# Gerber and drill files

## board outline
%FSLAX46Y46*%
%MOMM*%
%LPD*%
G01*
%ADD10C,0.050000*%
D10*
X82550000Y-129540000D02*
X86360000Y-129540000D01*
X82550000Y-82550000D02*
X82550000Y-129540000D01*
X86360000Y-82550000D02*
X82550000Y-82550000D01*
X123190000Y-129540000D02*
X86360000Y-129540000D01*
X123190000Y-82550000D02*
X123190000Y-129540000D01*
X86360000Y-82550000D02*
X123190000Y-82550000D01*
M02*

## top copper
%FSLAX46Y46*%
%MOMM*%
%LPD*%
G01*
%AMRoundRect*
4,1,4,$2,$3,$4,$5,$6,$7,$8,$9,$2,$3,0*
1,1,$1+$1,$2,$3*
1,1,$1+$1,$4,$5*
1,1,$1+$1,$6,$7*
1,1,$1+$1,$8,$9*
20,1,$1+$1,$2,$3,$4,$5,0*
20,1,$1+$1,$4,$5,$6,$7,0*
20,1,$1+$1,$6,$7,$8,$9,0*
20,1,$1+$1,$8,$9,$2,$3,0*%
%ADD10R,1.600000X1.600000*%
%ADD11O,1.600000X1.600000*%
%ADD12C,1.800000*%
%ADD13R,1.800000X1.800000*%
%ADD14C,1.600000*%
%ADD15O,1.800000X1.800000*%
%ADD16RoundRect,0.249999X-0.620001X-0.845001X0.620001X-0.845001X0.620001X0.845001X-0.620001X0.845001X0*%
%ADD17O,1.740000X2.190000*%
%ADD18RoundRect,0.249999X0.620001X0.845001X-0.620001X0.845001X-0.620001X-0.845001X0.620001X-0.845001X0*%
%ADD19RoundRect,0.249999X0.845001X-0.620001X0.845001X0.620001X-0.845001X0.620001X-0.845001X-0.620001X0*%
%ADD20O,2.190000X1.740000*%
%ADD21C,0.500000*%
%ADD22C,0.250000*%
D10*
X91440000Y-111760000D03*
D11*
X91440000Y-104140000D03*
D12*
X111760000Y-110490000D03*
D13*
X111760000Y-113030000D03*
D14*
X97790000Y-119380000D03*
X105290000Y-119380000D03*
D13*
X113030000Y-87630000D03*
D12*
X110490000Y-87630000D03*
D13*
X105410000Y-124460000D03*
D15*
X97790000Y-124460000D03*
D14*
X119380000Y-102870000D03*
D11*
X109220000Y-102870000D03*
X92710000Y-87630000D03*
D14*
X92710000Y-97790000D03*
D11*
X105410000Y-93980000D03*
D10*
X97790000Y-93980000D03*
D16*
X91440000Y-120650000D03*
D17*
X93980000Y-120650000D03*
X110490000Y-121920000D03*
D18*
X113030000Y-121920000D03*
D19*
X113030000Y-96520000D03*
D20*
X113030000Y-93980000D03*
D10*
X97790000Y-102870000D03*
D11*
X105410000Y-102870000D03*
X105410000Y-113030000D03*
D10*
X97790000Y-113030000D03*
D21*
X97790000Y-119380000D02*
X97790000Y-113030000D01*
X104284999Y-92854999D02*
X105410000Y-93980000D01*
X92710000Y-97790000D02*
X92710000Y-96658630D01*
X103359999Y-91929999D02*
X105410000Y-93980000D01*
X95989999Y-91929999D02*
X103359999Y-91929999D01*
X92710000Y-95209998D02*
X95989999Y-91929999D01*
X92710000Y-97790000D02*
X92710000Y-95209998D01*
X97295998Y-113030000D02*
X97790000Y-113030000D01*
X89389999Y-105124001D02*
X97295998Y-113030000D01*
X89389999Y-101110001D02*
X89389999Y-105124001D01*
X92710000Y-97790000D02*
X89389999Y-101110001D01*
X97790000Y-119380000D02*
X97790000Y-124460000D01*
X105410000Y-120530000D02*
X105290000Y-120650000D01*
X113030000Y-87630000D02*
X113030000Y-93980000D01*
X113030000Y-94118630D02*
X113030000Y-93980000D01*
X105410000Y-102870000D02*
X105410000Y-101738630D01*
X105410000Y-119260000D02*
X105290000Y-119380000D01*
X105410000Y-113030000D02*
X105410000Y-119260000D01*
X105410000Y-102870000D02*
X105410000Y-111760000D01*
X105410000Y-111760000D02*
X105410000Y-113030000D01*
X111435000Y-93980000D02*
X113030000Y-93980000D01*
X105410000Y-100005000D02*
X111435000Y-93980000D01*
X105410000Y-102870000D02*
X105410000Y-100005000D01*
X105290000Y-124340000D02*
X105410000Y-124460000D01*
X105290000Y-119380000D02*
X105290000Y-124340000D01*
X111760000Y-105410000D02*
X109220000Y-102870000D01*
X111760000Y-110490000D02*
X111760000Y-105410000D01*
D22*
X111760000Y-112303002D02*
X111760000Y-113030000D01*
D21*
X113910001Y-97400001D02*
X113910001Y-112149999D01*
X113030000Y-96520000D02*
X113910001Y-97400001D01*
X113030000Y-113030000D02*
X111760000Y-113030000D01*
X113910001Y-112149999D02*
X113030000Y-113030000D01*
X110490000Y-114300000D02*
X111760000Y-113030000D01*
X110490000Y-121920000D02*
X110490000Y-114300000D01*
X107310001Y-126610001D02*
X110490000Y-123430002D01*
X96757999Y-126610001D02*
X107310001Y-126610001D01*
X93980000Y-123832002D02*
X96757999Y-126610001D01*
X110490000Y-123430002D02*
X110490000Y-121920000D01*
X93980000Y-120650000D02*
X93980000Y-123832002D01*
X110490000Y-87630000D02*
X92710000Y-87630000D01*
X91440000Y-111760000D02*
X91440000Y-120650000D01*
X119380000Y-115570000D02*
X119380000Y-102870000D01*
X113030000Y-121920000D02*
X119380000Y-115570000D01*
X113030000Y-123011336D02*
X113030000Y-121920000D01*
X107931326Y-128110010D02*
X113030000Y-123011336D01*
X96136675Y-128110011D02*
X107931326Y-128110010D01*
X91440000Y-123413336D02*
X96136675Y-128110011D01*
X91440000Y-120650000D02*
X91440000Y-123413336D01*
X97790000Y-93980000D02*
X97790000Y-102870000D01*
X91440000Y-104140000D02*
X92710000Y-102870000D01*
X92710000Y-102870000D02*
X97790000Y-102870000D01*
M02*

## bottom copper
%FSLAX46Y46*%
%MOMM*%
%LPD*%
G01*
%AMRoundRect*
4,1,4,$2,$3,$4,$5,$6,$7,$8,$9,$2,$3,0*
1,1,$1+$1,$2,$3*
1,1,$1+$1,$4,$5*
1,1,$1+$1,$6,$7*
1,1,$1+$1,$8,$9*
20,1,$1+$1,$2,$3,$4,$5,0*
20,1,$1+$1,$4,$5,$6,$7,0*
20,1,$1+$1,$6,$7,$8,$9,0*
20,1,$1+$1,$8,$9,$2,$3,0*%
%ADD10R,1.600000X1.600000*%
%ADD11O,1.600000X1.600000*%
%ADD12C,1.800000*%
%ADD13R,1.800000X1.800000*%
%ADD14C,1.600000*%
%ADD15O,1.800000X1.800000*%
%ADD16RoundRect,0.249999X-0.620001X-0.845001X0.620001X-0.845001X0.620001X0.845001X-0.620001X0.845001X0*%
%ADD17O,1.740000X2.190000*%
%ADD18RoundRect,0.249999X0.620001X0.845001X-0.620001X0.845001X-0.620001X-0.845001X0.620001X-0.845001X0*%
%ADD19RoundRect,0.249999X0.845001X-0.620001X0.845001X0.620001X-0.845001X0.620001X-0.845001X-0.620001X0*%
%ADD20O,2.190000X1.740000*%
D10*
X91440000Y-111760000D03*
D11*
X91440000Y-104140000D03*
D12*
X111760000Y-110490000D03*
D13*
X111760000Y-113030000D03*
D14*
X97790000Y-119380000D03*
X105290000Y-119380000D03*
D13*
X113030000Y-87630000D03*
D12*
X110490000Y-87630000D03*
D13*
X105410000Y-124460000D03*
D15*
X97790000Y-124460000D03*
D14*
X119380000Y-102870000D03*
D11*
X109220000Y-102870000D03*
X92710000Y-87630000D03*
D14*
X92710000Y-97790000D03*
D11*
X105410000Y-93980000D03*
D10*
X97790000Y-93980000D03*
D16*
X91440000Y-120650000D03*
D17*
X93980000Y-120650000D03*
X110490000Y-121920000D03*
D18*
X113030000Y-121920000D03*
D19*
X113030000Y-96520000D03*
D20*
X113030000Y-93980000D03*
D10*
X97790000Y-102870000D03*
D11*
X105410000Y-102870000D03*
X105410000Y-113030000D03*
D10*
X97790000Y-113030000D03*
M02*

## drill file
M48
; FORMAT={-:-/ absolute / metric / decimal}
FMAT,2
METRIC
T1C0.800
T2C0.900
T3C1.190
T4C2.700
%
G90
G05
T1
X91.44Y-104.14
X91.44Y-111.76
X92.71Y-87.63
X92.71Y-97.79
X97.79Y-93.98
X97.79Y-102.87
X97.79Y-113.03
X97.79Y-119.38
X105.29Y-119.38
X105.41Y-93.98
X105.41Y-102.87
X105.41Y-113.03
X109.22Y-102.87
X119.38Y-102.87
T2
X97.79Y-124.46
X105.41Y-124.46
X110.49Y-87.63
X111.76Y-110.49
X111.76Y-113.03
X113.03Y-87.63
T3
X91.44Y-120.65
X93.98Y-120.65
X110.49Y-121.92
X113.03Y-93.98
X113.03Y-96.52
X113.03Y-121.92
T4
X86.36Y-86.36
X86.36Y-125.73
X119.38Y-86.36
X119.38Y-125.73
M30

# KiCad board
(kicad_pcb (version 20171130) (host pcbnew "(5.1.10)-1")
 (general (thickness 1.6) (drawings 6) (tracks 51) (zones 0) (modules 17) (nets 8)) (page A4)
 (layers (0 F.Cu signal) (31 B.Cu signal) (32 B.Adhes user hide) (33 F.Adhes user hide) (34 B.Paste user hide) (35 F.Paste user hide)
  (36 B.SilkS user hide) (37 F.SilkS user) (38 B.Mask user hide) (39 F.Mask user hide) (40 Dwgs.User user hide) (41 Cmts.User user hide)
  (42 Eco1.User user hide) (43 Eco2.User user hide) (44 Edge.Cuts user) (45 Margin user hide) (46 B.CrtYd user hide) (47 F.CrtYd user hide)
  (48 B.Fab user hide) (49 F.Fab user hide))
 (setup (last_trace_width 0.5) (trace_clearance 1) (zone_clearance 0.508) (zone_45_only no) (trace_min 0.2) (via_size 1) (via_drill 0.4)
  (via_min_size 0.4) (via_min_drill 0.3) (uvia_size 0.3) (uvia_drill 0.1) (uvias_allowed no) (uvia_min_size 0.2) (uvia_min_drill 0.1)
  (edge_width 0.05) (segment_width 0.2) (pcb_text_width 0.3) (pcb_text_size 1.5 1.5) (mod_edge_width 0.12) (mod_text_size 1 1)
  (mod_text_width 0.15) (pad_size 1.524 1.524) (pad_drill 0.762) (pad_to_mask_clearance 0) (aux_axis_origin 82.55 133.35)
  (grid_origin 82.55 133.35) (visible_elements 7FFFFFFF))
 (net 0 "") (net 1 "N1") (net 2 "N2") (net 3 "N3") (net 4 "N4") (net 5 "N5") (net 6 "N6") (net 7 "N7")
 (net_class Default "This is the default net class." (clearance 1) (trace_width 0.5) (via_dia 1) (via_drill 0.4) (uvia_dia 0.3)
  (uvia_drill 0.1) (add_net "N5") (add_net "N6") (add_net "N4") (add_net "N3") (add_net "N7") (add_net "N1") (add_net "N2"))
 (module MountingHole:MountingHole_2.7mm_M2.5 (layer F.Cu) (at 86.36 125.73)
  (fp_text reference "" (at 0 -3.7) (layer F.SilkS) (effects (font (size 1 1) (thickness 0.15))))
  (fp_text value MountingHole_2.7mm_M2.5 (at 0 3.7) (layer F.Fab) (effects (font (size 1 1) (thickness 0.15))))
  (pad 1 np_thru_hole circle (at 0 0) (size 2.7 2.7) (drill 2.7) (layers *.Cu *.Mask)))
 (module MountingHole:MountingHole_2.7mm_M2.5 (layer F.Cu) (at 86.36 86.36)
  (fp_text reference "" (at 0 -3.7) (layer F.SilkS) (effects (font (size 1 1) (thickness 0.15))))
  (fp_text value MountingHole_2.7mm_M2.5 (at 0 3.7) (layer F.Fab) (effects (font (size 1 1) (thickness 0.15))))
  (pad 1 np_thru_hole circle (at 0 0) (size 2.7 2.7) (drill 2.7) (layers *.Cu *.Mask)))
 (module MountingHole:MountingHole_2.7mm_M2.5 (layer F.Cu) (at 119.38 125.73)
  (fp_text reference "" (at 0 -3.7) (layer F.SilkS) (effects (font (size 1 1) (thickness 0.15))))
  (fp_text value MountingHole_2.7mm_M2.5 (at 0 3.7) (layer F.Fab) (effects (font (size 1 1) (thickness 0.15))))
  (pad 1 np_thru_hole circle (at 0 0) (size 2.7 2.7) (drill 2.7) (layers *.Cu *.Mask)))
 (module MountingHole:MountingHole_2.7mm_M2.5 (layer F.Cu) (at 119.38 86.36)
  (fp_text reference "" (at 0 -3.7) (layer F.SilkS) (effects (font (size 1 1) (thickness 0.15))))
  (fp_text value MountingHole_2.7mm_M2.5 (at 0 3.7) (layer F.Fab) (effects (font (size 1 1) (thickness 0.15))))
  (pad 1 np_thru_hole circle (at 0 0) (size 2.7 2.7) (drill 2.7) (layers *.Cu *.Mask)))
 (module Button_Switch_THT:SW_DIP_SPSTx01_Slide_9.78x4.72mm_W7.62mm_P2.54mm (layer F.Cu) (at 91.44 111.76 90)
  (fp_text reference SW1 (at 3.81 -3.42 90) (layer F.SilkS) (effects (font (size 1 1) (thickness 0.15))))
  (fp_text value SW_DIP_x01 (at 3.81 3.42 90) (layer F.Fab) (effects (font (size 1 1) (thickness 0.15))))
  (pad 1 thru_hole rect (at 0 0 90) (size 1.6 1.6) (drill 0.8) (layers *.Cu *.Mask) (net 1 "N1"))
  (pad 2 thru_hole oval (at 7.62 0 90) (size 1.6 1.6) (drill 0.8) (layers *.Cu *.Mask) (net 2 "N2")))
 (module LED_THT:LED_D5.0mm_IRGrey (layer F.Cu) (at 111.76 113.03 90)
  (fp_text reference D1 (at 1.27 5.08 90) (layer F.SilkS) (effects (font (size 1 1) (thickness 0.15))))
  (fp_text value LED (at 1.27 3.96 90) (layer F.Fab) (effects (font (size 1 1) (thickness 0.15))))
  (pad 2 thru_hole circle (at 2.54 0 90) (size 1.8 1.8) (drill 0.9) (layers *.Cu *.Mask) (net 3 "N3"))
  (pad 1 thru_hole rect (at 0 0 90) (size 1.8 1.8) (drill 0.9) (layers *.Cu *.Mask) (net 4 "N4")))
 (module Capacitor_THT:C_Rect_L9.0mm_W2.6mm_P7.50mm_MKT (layer F.Cu) (at 97.79 119.38)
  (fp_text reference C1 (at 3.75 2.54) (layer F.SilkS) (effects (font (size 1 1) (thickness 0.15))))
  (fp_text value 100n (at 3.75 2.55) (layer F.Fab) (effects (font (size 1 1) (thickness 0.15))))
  (pad 1 thru_hole circle (at 0 0) (size 1.6 1.6) (drill 0.8) (layers *.Cu *.Mask) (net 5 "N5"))
  (pad 2 thru_hole circle (at 7.5 0) (size 1.6 1.6) (drill 0.8) (layers *.Cu *.Mask) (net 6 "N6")))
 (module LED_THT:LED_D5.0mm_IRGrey (layer F.Cu) (at 113.03 87.63 180)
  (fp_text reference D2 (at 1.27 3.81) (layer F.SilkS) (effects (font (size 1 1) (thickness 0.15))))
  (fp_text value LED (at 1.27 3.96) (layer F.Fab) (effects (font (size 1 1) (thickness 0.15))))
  (pad 1 thru_hole rect (at 0 0 180) (size 1.8 1.8) (drill 0.9) (layers *.Cu *.Mask) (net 6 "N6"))
  (pad 2 thru_hole circle (at 2.54 0 180) (size 1.8 1.8) (drill 0.9) (layers *.Cu *.Mask) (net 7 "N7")))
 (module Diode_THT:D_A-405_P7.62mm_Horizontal (layer F.Cu) (at 105.41 124.46 180)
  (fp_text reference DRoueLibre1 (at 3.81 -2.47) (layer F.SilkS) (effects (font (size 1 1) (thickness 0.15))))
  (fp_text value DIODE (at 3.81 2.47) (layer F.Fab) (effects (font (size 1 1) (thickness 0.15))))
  (pad 1 thru_hole rect (at 0 0 180) (size 1.8 1.8) (drill 0.9) (layers *.Cu *.Mask) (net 6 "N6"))
  (pad 2 thru_hole oval (at 7.62 0 180) (size 1.8 1.8) (drill 0.9) (layers *.Cu *.Mask) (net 5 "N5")))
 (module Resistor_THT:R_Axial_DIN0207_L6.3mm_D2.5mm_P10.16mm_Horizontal (layer F.Cu) (at 119.38 102.87 180)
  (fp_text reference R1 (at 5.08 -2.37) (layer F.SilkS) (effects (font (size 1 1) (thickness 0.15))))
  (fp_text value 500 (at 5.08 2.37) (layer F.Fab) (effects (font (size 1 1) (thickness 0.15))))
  (pad 1 thru_hole circle (at 0 0 180) (size 1.6 1.6) (drill 0.8) (layers *.Cu *.Mask) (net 1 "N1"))
  (pad 2 thru_hole oval (at 10.16 0 180) (size 1.6 1.6) (drill 0.8) (layers *.Cu *.Mask) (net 3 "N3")))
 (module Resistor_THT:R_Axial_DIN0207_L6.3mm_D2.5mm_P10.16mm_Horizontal (layer F.Cu) (at 92.71 97.79 90)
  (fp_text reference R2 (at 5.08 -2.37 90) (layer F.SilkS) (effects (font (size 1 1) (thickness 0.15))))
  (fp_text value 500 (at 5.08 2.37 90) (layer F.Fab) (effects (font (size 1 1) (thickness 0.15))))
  (pad 2 thru_hole oval (at 10.16 0 90) (size 1.6 1.6) (drill 0.8) (layers *.Cu *.Mask) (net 7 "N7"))
  (pad 1 thru_hole circle (at 0 0 90) (size 1.6 1.6) (drill 0.8) (layers *.Cu *.Mask) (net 5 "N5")))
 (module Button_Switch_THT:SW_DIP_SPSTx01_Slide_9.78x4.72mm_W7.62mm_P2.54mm (layer F.Cu) (at 97.79 93.98)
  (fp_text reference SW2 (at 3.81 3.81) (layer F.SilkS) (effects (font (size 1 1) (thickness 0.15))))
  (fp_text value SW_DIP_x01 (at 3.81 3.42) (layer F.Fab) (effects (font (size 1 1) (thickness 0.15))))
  (pad 2 thru_hole oval (at 7.62 0) (size 1.6 1.6) (drill 0.8) (layers *.Cu *.Mask) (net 5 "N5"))
  (pad 1 thru_hole rect (at 0 0) (size 1.6 1.6) (drill 0.8) (layers *.Cu *.Mask) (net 2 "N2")))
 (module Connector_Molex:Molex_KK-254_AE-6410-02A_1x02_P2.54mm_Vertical (layer F.Cu) (at 91.44 120.65)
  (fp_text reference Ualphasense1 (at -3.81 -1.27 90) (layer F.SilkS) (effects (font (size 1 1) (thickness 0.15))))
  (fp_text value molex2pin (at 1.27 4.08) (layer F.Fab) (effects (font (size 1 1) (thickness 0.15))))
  (pad 1 thru_hole roundrect (at 0 0) (size 1.74 2.19) (drill 1.19) (layers *.Cu *.Mask) (roundrect_rratio 0.1436775862068966) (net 1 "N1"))
  (pad 2 thru_hole oval (at 2.54 0) (size 1.74 2.19) (drill 1.19) (layers *.Cu *.Mask) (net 4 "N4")))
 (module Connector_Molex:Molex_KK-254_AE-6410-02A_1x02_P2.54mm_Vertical (layer F.Cu) (at 113.03 121.92 180)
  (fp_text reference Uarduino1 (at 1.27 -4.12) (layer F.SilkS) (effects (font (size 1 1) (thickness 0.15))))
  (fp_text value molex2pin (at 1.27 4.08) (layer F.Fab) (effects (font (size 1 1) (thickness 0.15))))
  (pad 2 thru_hole oval (at 2.54 0 180) (size 1.74 2.19) (drill 1.19) (layers *.Cu *.Mask) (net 4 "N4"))
  (pad 1 thru_hole roundrect (at 0 0 180) (size 1.74 2.19) (drill 1.19) (layers *.Cu *.Mask) (roundrect_rratio 0.1436775862068966)
   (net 1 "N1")))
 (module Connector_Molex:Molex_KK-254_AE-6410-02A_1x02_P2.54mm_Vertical (layer F.Cu) (at 113.03 96.52 90)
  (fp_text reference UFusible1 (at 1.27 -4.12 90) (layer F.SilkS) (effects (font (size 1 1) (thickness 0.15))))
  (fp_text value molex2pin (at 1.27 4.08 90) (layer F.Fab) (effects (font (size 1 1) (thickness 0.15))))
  (pad 1 thru_hole roundrect (at 0 0 90) (size 1.74 2.19) (drill 1.19) (layers *.Cu *.Mask) (roundrect_rratio 0.1436775862068966)
   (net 4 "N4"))
  (pad 2 thru_hole oval (at 2.54 0 90) (size 1.74 2.19) (drill 1.19) (layers *.Cu *.Mask) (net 6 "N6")))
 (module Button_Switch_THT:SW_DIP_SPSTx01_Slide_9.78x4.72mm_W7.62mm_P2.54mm (layer F.Cu) (at 97.79 102.87)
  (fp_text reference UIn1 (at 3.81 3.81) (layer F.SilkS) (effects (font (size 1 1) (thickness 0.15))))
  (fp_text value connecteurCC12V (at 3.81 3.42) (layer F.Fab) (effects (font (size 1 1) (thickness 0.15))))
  (pad 1 thru_hole rect (at 0 0) (size 1.6 1.6) (drill 0.8) (layers *.Cu *.Mask) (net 2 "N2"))
  (pad 2 thru_hole oval (at 7.62 0) (size 1.6 1.6) (drill 0.8) (layers *.Cu *.Mask) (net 6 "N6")))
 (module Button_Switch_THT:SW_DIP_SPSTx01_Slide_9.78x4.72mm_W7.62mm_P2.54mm (layer F.Cu) (at 97.79 113.03)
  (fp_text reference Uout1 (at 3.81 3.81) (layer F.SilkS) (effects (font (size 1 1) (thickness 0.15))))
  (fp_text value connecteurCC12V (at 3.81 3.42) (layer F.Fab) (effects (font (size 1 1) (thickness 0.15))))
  (pad 2 thru_hole oval (at 7.62 0) (size 1.6 1.6) (drill 0.8) (layers *.Cu *.Mask) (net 6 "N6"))
  (pad 1 thru_hole rect (at 0 0) (size 1.6 1.6) (drill 0.8) (layers *.Cu *.Mask) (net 5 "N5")))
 (gr_line (start 82.55 129.54) (end 86.36 129.54) (layer Edge.Cuts) (width 0.05))
 (gr_line (start 82.55 82.55) (end 82.55 129.54) (layer Edge.Cuts) (width 0.05))
 (gr_line (start 86.36 82.55) (end 82.55 82.55) (layer Edge.Cuts) (width 0.05))
 (gr_line (start 123.19 129.54) (end 86.36 129.54) (layer Edge.Cuts) (width 0.05))
 (gr_line (start 123.19 82.55) (end 123.19 129.54) (layer Edge.Cuts) (width 0.05))
 (gr_line (start 86.36 82.55) (end 123.19 82.55) (layer Edge.Cuts) (width 0.05))
 (segment (start 97.79 119.38) (end 97.79 113.03) (width 0.5) (layer F.Cu) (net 5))
 (segment (start 104.284999 92.854999) (end 105.41 93.98) (width 0.5) (layer F.Cu) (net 5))
 (segment (start 92.71 97.79) (end 92.71 96.65863) (width 0.5) (layer F.Cu) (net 5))
 (segment (start 103.359999 91.929999) (end 105.41 93.98) (width 0.5) (layer F.Cu) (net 5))
 (segment (start 95.989999 91.929999) (end 103.359999 91.929999) (width 0.5) (layer F.Cu) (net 5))
 (segment (start 92.71 95.209998) (end 95.989999 91.929999) (width 0.5) (layer F.Cu) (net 5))
 (segment (start 92.71 97.79) (end 92.71 95.209998) (width 0.5) (layer F.Cu) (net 5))
 (segment (start 97.295998 113.03) (end 97.79 113.03) (width 0.5) (layer F.Cu) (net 5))
 (segment (start 89.389999 105.124001) (end 97.295998 113.03) (width 0.5) (layer F.Cu) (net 5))
 (segment (start 89.389999 101.110001) (end 89.389999 105.124001) (width 0.5) (layer F.Cu) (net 5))
 (segment (start 92.71 97.79) (end 89.389999 101.110001) (width 0.5) (layer F.Cu) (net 5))
 (segment (start 97.79 119.38) (end 97.79 124.46) (width 0.5) (layer F.Cu) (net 5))
 (segment (start 105.41 120.53) (end 105.29 120.65) (width 0.5) (layer F.Cu) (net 6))
 (segment (start 113.03 87.63) (end 113.03 93.98) (width 0.5) (layer F.Cu) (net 6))
 (segment (start 113.03 94.11863) (end 113.03 93.98) (width 0.5) (layer F.Cu) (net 6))
 (segment (start 105.41 102.87) (end 105.41 101.73863) (width 0.5) (layer F.Cu) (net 6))
 (segment (start 105.41 119.26) (end 105.29 119.38) (width 0.5) (layer F.Cu) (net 6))
 (segment (start 105.41 113.03) (end 105.41 119.26) (width 0.5) (layer F.Cu) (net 6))
 (segment (start 105.41 102.87) (end 105.41 111.76) (width 0.5) (layer F.Cu) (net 6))
 (segment (start 105.41 111.76) (end 105.41 113.03) (width 0.5) (layer F.Cu) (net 6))
 (segment (start 111.435 93.98) (end 113.03 93.98) (width 0.5) (layer F.Cu) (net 6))
 (segment (start 105.41 100.005) (end 111.435 93.98) (width 0.5) (layer F.Cu) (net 6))
 (segment (start 105.41 102.87) (end 105.41 100.005) (width 0.5) (layer F.Cu) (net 6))
 (segment (start 105.29 124.34) (end 105.41 124.46) (width 0.5) (layer F.Cu) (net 6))
 (segment (start 105.29 119.38) (end 105.29 124.34) (width 0.5) (layer F.Cu) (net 6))
 (segment (start 111.76 105.41) (end 109.22 102.87) (width 0.5) (layer F.Cu) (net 3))
 (segment (start 111.76 110.49) (end 111.76 105.41) (width 0.5) (layer F.Cu) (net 3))
 (segment (start 111.76 112.303002) (end 111.76 113.03) (width 0.25) (layer F.Cu) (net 4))
 (segment (start 113.910001 97.400001) (end 113.910001 112.149999) (width 0.5) (layer F.Cu) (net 4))
 (segment (start 113.03 96.52) (end 113.910001 97.400001) (width 0.5) (layer F.Cu) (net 4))
 (segment (start 113.03 113.03) (end 111.76 113.03) (width 0.5) (layer F.Cu) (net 4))
 (segment (start 113.910001 112.149999) (end 113.03 113.03) (width 0.5) (layer F.Cu) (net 4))
 (segment (start 110.49 114.3) (end 111.76 113.03) (width 0.5) (layer F.Cu) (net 4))
 (segment (start 110.49 121.92) (end 110.49 114.3) (width 0.5) (layer F.Cu) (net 4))
 (segment (start 107.310001 126.610001) (end 110.49 123.430002) (width 0.5) (layer F.Cu) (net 4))
 (segment (start 96.757999 126.610001) (end 107.310001 126.610001) (width 0.5) (layer F.Cu) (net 4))
 (segment (start 93.98 123.832002) (end 96.757999 126.610001) (width 0.5) (layer F.Cu) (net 4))
 (segment (start 110.49 123.430002) (end 110.49 121.92) (width 0.5) (layer F.Cu) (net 4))
 (segment (start 93.98 120.65) (end 93.98 123.832002) (width 0.5) (layer F.Cu) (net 4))
 (segment (start 110.49 87.63) (end 92.71 87.63) (width 0.5) (layer F.Cu) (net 7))
 (segment (start 91.44 111.76) (end 91.44 120.65) (width 0.5) (layer F.Cu) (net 1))
 (segment (start 119.38 115.57) (end 119.38 102.87) (width 0.5) (layer F.Cu) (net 1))
 (segment (start 113.03 121.92) (end 119.38 115.57) (width 0.5) (layer F.Cu) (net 1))
 (segment (start 113.03 123.011336) (end 113.03 121.92) (width 0.5) (layer F.Cu) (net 1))
 (segment (start 107.931326 128.11001) (end 113.03 123.011336) (width 0.5) (layer F.Cu) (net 1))
 (segment (start 96.136675 128.110011) (end 107.931326 128.11001) (width 0.5) (layer F.Cu) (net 1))
 (segment (start 91.44 123.413336) (end 96.136675 128.110011) (width 0.5) (layer F.Cu) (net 1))
 (segment (start 91.44 120.65) (end 91.44 123.413336) (width 0.5) (layer F.Cu) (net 1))
 (segment (start 97.79 93.98) (end 97.79 102.87) (width 0.5) (layer F.Cu) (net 2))
 (segment (start 91.44 104.14) (end 92.71 102.87) (width 0.5) (layer F.Cu) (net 2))
 (segment (start 92.71 102.87) (end 97.79 102.87) (width 0.5) (layer F.Cu) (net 2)))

